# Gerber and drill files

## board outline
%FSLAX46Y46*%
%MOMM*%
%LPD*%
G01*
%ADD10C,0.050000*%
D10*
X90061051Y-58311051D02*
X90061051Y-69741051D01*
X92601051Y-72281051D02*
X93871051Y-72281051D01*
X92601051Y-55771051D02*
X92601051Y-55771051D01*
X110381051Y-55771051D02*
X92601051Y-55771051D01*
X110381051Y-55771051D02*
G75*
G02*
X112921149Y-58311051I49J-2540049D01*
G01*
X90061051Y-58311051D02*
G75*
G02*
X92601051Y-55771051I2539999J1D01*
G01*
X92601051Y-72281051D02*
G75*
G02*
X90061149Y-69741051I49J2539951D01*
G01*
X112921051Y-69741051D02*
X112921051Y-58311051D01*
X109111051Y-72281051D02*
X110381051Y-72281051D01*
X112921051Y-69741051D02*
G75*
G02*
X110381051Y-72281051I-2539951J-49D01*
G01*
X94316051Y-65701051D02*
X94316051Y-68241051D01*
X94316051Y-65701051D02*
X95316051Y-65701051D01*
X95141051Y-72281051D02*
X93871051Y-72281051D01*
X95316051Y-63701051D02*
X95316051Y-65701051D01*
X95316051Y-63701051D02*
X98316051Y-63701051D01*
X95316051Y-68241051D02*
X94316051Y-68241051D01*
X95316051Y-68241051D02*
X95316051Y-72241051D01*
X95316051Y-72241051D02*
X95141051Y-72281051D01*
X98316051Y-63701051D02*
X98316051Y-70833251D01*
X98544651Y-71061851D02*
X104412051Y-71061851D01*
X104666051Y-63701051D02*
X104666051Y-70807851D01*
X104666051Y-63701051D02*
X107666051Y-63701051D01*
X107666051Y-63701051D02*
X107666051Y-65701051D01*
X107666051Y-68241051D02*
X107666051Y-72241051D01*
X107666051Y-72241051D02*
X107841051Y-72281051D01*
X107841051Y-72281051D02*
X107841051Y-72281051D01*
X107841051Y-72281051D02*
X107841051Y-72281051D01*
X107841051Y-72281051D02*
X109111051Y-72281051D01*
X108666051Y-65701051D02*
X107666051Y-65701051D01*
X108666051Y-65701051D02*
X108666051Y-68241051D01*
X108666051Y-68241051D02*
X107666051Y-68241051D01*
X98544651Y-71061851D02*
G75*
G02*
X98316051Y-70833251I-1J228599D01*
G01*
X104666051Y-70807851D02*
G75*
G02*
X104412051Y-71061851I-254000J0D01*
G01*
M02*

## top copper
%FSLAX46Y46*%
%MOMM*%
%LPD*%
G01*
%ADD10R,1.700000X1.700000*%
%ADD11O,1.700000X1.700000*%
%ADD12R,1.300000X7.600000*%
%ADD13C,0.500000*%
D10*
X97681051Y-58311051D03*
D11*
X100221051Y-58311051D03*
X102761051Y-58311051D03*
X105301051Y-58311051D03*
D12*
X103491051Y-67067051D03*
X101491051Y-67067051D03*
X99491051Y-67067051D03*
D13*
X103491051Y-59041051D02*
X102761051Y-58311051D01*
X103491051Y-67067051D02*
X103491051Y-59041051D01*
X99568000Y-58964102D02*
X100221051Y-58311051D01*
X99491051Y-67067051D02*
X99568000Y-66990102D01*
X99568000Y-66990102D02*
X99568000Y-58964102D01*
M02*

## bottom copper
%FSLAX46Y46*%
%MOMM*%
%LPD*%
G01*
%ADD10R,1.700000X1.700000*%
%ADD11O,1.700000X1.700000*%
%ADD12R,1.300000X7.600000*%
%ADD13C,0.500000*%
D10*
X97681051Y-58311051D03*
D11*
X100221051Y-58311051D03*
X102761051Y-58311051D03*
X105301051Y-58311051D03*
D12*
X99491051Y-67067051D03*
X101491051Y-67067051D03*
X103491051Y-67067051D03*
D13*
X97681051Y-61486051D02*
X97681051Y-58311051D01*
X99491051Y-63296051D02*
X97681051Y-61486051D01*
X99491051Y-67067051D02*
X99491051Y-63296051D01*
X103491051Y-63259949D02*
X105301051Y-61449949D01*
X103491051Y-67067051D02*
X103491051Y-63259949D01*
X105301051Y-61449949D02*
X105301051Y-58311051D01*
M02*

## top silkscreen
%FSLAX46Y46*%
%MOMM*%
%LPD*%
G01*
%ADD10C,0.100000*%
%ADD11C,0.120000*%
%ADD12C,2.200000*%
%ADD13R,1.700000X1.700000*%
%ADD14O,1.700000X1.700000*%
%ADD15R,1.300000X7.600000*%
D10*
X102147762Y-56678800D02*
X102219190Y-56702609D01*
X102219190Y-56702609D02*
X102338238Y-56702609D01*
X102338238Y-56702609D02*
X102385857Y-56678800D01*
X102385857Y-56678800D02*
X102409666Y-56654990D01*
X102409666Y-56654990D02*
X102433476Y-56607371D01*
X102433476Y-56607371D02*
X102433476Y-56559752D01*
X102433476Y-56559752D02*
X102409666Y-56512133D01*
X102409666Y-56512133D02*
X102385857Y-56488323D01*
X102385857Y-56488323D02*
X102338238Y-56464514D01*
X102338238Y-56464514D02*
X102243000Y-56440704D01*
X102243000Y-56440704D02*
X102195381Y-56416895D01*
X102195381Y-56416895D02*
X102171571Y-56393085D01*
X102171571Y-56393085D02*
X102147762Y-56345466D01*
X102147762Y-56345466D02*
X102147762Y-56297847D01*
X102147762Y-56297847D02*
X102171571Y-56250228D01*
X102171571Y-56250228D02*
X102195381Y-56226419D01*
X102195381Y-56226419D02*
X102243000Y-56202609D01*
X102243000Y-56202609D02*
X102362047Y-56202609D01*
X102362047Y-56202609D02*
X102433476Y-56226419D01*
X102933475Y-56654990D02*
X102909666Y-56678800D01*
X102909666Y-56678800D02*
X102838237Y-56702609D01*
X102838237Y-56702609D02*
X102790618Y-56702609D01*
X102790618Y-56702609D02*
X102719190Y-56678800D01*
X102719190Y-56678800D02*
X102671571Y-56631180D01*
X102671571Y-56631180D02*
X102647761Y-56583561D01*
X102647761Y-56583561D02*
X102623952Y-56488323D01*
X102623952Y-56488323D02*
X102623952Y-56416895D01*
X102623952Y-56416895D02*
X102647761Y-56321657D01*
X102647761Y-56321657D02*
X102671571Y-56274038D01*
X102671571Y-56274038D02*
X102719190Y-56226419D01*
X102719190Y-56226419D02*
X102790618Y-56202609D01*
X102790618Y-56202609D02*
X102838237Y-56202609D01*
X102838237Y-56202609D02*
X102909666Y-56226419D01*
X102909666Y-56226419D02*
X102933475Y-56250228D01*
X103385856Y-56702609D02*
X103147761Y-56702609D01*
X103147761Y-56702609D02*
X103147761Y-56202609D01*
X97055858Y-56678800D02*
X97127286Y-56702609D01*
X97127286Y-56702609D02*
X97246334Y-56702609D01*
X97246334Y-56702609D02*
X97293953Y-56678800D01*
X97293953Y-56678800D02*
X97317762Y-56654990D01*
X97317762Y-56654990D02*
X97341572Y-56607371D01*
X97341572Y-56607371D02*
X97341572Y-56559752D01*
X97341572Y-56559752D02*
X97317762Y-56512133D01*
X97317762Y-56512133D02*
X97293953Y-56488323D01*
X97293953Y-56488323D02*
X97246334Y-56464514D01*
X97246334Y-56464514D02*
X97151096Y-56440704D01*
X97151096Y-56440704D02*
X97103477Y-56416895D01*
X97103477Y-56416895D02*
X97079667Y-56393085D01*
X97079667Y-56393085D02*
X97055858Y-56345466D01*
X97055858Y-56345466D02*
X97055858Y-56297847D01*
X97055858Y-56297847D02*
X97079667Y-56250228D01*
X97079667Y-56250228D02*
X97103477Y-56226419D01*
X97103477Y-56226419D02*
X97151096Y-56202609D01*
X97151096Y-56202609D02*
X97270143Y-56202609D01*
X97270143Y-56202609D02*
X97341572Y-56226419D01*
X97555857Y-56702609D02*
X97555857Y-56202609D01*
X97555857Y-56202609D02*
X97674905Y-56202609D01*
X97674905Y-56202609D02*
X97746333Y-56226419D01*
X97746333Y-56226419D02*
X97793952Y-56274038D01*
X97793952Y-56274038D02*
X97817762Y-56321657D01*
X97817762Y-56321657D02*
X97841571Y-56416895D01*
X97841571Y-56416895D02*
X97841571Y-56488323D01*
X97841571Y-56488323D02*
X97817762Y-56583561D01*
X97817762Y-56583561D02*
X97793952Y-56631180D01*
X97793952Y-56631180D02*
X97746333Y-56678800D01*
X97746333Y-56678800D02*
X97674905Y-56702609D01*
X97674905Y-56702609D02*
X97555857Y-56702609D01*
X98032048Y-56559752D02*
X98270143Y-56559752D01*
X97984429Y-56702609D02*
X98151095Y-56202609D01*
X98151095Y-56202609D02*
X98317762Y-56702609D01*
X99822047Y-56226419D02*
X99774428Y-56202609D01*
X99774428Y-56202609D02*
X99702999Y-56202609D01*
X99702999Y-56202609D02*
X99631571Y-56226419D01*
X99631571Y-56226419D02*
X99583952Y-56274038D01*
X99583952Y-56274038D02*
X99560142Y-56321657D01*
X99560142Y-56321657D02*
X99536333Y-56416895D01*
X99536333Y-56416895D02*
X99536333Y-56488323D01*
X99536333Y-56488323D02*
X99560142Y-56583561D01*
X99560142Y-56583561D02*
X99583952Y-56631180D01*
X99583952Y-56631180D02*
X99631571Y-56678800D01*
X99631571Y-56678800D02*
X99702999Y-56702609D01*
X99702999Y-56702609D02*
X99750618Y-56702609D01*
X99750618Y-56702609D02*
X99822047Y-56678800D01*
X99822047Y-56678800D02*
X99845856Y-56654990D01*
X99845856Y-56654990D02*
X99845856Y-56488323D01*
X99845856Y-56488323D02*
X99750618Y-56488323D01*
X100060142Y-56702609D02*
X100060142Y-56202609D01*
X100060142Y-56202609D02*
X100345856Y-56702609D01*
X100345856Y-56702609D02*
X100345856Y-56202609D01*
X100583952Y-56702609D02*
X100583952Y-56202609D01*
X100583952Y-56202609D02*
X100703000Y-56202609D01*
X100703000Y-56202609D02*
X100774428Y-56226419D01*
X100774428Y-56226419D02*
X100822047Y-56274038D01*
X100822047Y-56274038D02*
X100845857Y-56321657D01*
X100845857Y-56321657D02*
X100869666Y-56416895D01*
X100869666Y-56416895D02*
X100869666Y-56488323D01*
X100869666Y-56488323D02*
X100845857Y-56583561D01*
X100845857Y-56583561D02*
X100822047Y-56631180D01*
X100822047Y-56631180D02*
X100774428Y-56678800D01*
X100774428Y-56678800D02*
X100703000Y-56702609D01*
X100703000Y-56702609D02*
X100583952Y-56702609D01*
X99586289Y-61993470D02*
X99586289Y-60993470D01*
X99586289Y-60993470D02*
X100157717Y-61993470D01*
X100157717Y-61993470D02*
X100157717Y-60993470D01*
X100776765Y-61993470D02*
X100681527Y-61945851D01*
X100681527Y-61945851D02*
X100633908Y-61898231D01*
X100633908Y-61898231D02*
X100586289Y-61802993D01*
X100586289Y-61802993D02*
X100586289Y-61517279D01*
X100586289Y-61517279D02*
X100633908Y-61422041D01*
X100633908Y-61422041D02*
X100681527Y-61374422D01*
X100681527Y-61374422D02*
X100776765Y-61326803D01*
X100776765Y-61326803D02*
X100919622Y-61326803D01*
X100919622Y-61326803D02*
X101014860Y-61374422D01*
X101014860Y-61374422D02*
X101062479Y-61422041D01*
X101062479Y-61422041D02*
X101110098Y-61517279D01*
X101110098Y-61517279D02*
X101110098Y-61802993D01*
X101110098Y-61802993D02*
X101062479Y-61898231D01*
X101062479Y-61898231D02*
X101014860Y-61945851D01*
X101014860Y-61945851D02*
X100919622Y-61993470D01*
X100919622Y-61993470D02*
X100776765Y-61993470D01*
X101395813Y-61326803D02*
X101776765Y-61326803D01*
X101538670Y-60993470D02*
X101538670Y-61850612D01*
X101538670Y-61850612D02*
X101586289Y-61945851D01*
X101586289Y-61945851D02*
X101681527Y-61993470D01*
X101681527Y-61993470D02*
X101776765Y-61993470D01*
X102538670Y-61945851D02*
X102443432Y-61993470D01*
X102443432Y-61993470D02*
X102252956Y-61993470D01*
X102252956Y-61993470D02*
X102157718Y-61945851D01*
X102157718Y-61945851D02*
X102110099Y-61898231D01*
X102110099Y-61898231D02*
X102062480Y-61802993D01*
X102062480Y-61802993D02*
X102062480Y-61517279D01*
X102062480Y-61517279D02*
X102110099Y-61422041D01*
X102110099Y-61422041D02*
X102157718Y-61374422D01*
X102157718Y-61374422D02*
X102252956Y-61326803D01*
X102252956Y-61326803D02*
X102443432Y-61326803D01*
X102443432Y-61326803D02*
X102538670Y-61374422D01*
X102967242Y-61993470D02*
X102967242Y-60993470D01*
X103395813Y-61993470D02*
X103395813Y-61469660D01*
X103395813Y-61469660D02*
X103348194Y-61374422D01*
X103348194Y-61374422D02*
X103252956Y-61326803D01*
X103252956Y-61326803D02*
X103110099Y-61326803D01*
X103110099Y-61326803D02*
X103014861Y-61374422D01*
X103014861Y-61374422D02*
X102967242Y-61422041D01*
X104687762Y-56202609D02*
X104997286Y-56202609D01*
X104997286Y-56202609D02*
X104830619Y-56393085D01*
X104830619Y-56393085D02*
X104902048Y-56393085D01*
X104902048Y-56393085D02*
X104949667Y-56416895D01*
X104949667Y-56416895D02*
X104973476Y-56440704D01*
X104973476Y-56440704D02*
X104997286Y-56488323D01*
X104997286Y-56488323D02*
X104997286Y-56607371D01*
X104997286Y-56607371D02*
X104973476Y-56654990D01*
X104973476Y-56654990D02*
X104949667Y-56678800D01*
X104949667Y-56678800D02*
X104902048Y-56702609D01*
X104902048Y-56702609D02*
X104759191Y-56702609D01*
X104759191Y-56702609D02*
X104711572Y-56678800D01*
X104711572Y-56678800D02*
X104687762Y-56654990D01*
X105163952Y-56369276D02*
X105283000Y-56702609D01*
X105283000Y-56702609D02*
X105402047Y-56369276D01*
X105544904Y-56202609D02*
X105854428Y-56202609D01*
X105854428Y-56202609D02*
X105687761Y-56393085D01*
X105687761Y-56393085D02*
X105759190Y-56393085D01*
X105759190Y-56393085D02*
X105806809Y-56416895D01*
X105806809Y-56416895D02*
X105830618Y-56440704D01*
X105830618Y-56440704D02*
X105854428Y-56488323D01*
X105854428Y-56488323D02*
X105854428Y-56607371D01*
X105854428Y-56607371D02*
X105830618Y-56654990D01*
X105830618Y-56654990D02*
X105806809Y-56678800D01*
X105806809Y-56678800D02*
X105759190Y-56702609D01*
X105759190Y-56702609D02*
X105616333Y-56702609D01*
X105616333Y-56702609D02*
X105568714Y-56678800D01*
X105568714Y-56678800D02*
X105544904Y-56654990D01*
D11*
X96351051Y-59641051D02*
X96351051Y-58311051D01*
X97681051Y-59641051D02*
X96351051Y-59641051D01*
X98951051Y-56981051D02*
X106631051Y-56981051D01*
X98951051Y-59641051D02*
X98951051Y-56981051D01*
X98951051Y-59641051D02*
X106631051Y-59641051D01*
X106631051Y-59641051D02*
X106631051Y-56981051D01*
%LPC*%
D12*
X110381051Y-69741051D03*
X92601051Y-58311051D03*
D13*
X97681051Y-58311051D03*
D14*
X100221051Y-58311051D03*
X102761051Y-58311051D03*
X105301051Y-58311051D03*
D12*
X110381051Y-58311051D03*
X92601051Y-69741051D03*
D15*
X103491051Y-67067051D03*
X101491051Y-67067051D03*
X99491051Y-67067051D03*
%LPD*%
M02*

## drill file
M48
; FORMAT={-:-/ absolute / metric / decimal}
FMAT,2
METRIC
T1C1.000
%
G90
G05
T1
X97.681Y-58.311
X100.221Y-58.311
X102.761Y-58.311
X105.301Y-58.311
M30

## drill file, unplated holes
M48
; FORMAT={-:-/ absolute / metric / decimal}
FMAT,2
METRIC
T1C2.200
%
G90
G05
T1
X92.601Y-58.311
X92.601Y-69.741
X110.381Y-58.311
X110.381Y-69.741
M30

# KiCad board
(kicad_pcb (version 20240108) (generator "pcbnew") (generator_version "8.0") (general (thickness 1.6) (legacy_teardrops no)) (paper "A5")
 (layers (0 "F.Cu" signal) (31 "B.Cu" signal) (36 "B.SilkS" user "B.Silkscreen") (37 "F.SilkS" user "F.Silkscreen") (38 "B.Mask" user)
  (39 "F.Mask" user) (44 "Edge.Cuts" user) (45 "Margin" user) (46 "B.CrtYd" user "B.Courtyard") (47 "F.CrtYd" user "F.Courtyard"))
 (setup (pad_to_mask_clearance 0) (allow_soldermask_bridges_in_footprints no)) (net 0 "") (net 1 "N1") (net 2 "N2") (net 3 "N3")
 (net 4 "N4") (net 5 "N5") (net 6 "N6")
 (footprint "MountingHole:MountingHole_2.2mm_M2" (layer "F.Cu") (at 110.381051 69.741051)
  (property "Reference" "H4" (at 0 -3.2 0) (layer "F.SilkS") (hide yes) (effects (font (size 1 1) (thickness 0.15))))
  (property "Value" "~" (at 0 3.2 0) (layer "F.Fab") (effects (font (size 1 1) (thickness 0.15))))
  (pad "" np_thru_hole circle (at 0 0) (size 2.2 2.2) (drill 2.2) (layers "*.Cu" "*.Mask")))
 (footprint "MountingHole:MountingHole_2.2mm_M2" (layer "F.Cu") (at 92.601051 58.311051)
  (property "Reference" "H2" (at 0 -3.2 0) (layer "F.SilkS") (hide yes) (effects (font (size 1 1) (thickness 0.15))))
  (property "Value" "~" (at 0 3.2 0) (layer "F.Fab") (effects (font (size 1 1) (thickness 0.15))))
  (pad "" np_thru_hole circle (at 0 0) (size 2.2 2.2) (drill 2.2) (layers "*.Cu" "*.Mask")))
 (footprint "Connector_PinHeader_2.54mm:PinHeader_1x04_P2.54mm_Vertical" (layer "F.Cu") (at 97.681051 58.311051 90)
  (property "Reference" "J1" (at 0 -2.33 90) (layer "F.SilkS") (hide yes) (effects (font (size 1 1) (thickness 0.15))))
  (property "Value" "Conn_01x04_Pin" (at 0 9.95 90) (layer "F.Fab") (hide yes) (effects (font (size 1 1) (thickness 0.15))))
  (fp_line (start -1.33 -1.33) (end 0 -1.33) (stroke (width 0.12) (type solid)) (layer "F.SilkS"))
  (fp_line (start -1.33 0) (end -1.33 -1.33) (stroke (width 0.12) (type solid)) (layer "F.SilkS"))
  (fp_line (start 1.33 1.27) (end 1.33 8.95) (stroke (width 0.12) (type solid)) (layer "F.SilkS"))
  (fp_line (start -1.33 1.27) (end 1.33 1.27) (stroke (width 0.12) (type solid)) (layer "F.SilkS"))
  (fp_line (start -1.33 1.27) (end -1.33 8.95) (stroke (width 0.12) (type solid)) (layer "F.SilkS"))
  (fp_line (start -1.33 8.95) (end 1.33 8.95) (stroke (width 0.12) (type solid)) (layer "F.SilkS"))
  (pad "1" thru_hole rect (at 0 0 90) (size 1.7 1.7) (drill 1) (layers "*.Cu" "*.Mask") (remove_unused_layers no) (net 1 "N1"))
  (pad "2" thru_hole oval (at 0 2.54 90) (size 1.7 1.7) (drill 1) (layers "*.Cu" "*.Mask") (remove_unused_layers no) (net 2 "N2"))
  (pad "3" thru_hole oval (at 0 5.08 90) (size 1.7 1.7) (drill 1) (layers "*.Cu" "*.Mask") (remove_unused_layers no) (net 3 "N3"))
  (pad "4" thru_hole oval (at 0 7.62 90) (size 1.7 1.7) (drill 1) (layers "*.Cu" "*.Mask") (remove_unused_layers no) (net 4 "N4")))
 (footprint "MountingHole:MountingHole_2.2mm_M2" (layer "F.Cu") (at 110.381051 58.311051)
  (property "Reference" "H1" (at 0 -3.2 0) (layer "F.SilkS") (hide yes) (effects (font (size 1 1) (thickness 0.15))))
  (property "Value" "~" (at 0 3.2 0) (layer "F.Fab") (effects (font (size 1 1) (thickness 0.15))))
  (pad "" np_thru_hole circle (at 0 0) (size 2.2 2.2) (drill 2.2) (layers "*.Cu" "*.Mask")))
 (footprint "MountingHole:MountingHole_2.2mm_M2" (layer "F.Cu") (at 92.601051 69.741051)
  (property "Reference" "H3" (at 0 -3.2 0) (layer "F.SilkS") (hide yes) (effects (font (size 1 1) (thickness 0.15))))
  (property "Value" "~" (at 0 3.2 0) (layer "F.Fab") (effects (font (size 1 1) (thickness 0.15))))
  (pad "" np_thru_hole circle (at 0 0) (size 2.2 2.2) (drill 2.2) (layers "*.Cu" "*.Mask")))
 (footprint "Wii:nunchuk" (layer "F.Cu") (at 101.491051 67.201051)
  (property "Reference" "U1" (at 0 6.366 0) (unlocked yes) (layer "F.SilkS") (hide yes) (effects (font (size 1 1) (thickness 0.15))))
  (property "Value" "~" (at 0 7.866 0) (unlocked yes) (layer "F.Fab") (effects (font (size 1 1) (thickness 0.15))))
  (fp_line (start -7.175 -1.5) (end -7.175 1.04) (stroke (width 0.05) (type default)) (layer "Edge.Cuts"))
  (fp_line (start -7.175 -1.5) (end -6.175 -1.5) (stroke (width 0.05) (type default)) (layer "Edge.Cuts"))
  (fp_line (start -6.35 5.08) (end -7.62 5.08) (stroke (width 0.05) (type default)) (layer "Edge.Cuts"))
  (fp_line (start -6.175 -3.5) (end -6.175 -1.5) (stroke (width 0.05) (type default)) (layer "Edge.Cuts"))
  (fp_line (start -6.175 -3.5) (end -3.175 -3.5) (stroke (width 0.05) (type default)) (layer "Edge.Cuts"))
  (fp_line (start -6.175 1.04) (end -7.175 1.04) (stroke (width 0.05) (type default)) (layer "Edge.Cuts"))
  (fp_line (start -6.175 1.04) (end -6.175 5.04) (stroke (width 0.05) (type default)) (layer "Edge.Cuts"))
  (fp_line (start -6.175 5.04) (end -6.35 5.08) (stroke (width 0.05) (type default)) (layer "Edge.Cuts"))
  (fp_line (start -3.175 -3.5) (end -3.175 3.6322) (stroke (width 0.05) (type default)) (layer "Edge.Cuts"))
  (fp_line (start -2.9464 3.8608) (end 2.921 3.8608) (stroke (width 0.05) (type default)) (layer "Edge.Cuts"))
  (fp_line (start 3.175 -3.5) (end 3.175 3.6068) (stroke (width 0.05) (type default)) (layer "Edge.Cuts"))
  (fp_line (start 3.175 -3.5) (end 6.175 -3.5) (stroke (width 0.05) (type default)) (layer "Edge.Cuts"))
  (fp_line (start 6.175 -3.5) (end 6.175 -1.5) (stroke (width 0.05) (type default)) (layer "Edge.Cuts"))
  (fp_line (start 6.175 1.04) (end 6.175 5.04) (stroke (width 0.05) (type default)) (layer "Edge.Cuts"))
  (fp_line (start 6.175 5.04) (end 6.35 5.08) (stroke (width 0.05) (type default)) (layer "Edge.Cuts"))
  (fp_line (start 6.35 5.08) (end 6.35 5.08) (stroke (width 0.05) (type default)) (layer "Edge.Cuts"))
  (fp_line (start 6.35 5.08) (end 6.35 5.08) (stroke (width 0.05) (type default)) (layer "Edge.Cuts"))
  (fp_line (start 6.35 5.08) (end 7.62 5.08) (stroke (width 0.05) (type default)) (layer "Edge.Cuts"))
  (fp_line (start 7.175 -1.5) (end 6.175 -1.5) (stroke (width 0.05) (type default)) (layer "Edge.Cuts"))
  (fp_line (start 7.175 -1.5) (end 7.175 1.04) (stroke (width 0.05) (type default)) (layer "Edge.Cuts"))
  (fp_line (start 7.175 1.04) (end 6.175 1.04) (stroke (width 0.05) (type default)) (layer "Edge.Cuts"))
  (fp_arc (start -2.9464 3.8608) (mid -3.108045 3.793845) (end -3.175 3.6322) (stroke (width 0.05) (type default)) (layer "Edge.Cuts"))
  (fp_arc (start 3.175 3.6068) (mid 3.100605 3.786405) (end 2.921 3.8608) (stroke (width 0.05) (type default)) (layer "Edge.Cuts"))
  (pad "1" smd rect (at -2 -0.134 270) (size 7.6 1.3) (layers "B.Cu" "B.Paste" "B.Mask") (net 1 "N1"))
  (pad "2" smd rect (at 0 -0.134 270) (size 7.6 1.3) (layers "B.Cu" "B.Paste" "B.Mask") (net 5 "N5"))
  (pad "3" smd rect (at 2 -0.134 270) (size 7.6 1.3) (layers "B.Cu" "B.Paste" "B.Mask") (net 4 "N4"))
  (pad "4" smd rect (at 2 -0.134 90) (size 7.6 1.3) (layers "F.Cu" "F.Paste" "F.Mask") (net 3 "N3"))
  (pad "5" smd rect (at 0 -0.134 90) (size 7.6 1.3) (layers "F.Cu" "F.Paste" "F.Mask") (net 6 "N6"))
  (pad "6" smd rect (at -2 -0.134 90) (size 7.6 1.3) (layers "F.Cu" "F.Paste" "F.Mask") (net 2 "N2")))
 (gr_line (start 90.061051 58.311051) (end 90.061051 69.741051) (stroke (width 0.05) (type default)) (layer "Edge.Cuts"))
 (gr_line (start 92.601051 72.281051) (end 93.871051 72.281051) (stroke (width 0.05) (type default)) (layer "Edge.Cuts"))
 (gr_line (start 92.601051 55.771051) (end 92.601051 55.771051) (stroke (width 0.05) (type default)) (layer "Edge.Cuts"))
 (gr_line (start 110.381051 55.771051) (end 92.601051 55.771051) (stroke (width 0.05) (type default)) (layer "Edge.Cuts"))
 (gr_arc (start 110.381051 55.771051) (mid 112.177102 56.515) (end 112.921051 58.311051) (stroke (width 0.05) (type default))
  (layer "Edge.Cuts"))
 (gr_arc (start 90.061051 58.311051) (mid 90.805 56.515) (end 92.601051 55.771051) (stroke (width 0.05) (type default)) (layer "Edge.Cuts"))
 (gr_arc (start 92.601051 72.281051) (mid 90.805 71.537102) (end 90.061051 69.741051) (stroke (width 0.05) (type default))
  (layer "Edge.Cuts"))
 (gr_line (start 112.921051 69.741051) (end 112.921051 58.311051) (stroke (width 0.05) (type default)) (layer "Edge.Cuts"))
 (gr_line (start 109.111051 72.281051) (end 110.381051 72.281051) (stroke (width 0.05) (type default)) (layer "Edge.Cuts"))
 (gr_arc (start 112.921051 69.741051) (mid 112.177102 71.537102) (end 110.381051 72.281051) (stroke (width 0.05) (type default))
  (layer "Edge.Cuts"))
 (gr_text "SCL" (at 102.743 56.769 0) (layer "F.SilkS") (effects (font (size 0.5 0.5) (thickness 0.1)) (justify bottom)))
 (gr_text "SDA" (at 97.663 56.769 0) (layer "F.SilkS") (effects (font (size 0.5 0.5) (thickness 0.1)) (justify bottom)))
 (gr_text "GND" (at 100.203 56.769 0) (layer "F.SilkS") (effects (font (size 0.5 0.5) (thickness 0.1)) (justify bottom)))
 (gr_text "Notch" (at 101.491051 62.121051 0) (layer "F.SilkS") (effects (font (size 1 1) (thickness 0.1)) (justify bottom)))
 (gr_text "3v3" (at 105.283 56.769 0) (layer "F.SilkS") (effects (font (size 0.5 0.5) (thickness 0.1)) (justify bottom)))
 (segment (start 97.681051 61.486051) (end 97.681051 58.311051) (width 0.5) (layer "B.Cu") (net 1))
 (segment (start 99.491051 63.296051) (end 97.681051 61.486051) (width 0.5) (layer "B.Cu") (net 1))
 (segment (start 99.491051 67.067051) (end 99.491051 63.296051) (width 0.5) (layer "B.Cu") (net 1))
 (segment (start 103.491051 59.041051) (end 102.761051 58.311051) (width 0.5) (layer "F.Cu") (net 3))
 (segment (start 103.491051 67.067051) (end 103.491051 59.041051) (width 0.5) (layer "F.Cu") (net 3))
 (segment (start 99.568 58.964102) (end 100.221051 58.311051) (width 0.5) (layer "F.Cu") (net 2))
 (segment (start 99.491051 67.067051) (end 99.568 66.990102) (width 0.5) (layer "F.Cu") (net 2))
 (segment (start 99.568 66.990102) (end 99.568 58.964102) (width 0.5) (layer "F.Cu") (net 2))
 (segment (start 103.491051 63.259949) (end 105.301051 61.449949) (width 0.5) (layer "B.Cu") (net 4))
 (segment (start 103.491051 67.067051) (end 103.491051 63.259949) (width 0.5) (layer "B.Cu") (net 4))
 (segment (start 105.301051 61.449949) (end 105.301051 58.311051) (width 0.5) (layer "B.Cu") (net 4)))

